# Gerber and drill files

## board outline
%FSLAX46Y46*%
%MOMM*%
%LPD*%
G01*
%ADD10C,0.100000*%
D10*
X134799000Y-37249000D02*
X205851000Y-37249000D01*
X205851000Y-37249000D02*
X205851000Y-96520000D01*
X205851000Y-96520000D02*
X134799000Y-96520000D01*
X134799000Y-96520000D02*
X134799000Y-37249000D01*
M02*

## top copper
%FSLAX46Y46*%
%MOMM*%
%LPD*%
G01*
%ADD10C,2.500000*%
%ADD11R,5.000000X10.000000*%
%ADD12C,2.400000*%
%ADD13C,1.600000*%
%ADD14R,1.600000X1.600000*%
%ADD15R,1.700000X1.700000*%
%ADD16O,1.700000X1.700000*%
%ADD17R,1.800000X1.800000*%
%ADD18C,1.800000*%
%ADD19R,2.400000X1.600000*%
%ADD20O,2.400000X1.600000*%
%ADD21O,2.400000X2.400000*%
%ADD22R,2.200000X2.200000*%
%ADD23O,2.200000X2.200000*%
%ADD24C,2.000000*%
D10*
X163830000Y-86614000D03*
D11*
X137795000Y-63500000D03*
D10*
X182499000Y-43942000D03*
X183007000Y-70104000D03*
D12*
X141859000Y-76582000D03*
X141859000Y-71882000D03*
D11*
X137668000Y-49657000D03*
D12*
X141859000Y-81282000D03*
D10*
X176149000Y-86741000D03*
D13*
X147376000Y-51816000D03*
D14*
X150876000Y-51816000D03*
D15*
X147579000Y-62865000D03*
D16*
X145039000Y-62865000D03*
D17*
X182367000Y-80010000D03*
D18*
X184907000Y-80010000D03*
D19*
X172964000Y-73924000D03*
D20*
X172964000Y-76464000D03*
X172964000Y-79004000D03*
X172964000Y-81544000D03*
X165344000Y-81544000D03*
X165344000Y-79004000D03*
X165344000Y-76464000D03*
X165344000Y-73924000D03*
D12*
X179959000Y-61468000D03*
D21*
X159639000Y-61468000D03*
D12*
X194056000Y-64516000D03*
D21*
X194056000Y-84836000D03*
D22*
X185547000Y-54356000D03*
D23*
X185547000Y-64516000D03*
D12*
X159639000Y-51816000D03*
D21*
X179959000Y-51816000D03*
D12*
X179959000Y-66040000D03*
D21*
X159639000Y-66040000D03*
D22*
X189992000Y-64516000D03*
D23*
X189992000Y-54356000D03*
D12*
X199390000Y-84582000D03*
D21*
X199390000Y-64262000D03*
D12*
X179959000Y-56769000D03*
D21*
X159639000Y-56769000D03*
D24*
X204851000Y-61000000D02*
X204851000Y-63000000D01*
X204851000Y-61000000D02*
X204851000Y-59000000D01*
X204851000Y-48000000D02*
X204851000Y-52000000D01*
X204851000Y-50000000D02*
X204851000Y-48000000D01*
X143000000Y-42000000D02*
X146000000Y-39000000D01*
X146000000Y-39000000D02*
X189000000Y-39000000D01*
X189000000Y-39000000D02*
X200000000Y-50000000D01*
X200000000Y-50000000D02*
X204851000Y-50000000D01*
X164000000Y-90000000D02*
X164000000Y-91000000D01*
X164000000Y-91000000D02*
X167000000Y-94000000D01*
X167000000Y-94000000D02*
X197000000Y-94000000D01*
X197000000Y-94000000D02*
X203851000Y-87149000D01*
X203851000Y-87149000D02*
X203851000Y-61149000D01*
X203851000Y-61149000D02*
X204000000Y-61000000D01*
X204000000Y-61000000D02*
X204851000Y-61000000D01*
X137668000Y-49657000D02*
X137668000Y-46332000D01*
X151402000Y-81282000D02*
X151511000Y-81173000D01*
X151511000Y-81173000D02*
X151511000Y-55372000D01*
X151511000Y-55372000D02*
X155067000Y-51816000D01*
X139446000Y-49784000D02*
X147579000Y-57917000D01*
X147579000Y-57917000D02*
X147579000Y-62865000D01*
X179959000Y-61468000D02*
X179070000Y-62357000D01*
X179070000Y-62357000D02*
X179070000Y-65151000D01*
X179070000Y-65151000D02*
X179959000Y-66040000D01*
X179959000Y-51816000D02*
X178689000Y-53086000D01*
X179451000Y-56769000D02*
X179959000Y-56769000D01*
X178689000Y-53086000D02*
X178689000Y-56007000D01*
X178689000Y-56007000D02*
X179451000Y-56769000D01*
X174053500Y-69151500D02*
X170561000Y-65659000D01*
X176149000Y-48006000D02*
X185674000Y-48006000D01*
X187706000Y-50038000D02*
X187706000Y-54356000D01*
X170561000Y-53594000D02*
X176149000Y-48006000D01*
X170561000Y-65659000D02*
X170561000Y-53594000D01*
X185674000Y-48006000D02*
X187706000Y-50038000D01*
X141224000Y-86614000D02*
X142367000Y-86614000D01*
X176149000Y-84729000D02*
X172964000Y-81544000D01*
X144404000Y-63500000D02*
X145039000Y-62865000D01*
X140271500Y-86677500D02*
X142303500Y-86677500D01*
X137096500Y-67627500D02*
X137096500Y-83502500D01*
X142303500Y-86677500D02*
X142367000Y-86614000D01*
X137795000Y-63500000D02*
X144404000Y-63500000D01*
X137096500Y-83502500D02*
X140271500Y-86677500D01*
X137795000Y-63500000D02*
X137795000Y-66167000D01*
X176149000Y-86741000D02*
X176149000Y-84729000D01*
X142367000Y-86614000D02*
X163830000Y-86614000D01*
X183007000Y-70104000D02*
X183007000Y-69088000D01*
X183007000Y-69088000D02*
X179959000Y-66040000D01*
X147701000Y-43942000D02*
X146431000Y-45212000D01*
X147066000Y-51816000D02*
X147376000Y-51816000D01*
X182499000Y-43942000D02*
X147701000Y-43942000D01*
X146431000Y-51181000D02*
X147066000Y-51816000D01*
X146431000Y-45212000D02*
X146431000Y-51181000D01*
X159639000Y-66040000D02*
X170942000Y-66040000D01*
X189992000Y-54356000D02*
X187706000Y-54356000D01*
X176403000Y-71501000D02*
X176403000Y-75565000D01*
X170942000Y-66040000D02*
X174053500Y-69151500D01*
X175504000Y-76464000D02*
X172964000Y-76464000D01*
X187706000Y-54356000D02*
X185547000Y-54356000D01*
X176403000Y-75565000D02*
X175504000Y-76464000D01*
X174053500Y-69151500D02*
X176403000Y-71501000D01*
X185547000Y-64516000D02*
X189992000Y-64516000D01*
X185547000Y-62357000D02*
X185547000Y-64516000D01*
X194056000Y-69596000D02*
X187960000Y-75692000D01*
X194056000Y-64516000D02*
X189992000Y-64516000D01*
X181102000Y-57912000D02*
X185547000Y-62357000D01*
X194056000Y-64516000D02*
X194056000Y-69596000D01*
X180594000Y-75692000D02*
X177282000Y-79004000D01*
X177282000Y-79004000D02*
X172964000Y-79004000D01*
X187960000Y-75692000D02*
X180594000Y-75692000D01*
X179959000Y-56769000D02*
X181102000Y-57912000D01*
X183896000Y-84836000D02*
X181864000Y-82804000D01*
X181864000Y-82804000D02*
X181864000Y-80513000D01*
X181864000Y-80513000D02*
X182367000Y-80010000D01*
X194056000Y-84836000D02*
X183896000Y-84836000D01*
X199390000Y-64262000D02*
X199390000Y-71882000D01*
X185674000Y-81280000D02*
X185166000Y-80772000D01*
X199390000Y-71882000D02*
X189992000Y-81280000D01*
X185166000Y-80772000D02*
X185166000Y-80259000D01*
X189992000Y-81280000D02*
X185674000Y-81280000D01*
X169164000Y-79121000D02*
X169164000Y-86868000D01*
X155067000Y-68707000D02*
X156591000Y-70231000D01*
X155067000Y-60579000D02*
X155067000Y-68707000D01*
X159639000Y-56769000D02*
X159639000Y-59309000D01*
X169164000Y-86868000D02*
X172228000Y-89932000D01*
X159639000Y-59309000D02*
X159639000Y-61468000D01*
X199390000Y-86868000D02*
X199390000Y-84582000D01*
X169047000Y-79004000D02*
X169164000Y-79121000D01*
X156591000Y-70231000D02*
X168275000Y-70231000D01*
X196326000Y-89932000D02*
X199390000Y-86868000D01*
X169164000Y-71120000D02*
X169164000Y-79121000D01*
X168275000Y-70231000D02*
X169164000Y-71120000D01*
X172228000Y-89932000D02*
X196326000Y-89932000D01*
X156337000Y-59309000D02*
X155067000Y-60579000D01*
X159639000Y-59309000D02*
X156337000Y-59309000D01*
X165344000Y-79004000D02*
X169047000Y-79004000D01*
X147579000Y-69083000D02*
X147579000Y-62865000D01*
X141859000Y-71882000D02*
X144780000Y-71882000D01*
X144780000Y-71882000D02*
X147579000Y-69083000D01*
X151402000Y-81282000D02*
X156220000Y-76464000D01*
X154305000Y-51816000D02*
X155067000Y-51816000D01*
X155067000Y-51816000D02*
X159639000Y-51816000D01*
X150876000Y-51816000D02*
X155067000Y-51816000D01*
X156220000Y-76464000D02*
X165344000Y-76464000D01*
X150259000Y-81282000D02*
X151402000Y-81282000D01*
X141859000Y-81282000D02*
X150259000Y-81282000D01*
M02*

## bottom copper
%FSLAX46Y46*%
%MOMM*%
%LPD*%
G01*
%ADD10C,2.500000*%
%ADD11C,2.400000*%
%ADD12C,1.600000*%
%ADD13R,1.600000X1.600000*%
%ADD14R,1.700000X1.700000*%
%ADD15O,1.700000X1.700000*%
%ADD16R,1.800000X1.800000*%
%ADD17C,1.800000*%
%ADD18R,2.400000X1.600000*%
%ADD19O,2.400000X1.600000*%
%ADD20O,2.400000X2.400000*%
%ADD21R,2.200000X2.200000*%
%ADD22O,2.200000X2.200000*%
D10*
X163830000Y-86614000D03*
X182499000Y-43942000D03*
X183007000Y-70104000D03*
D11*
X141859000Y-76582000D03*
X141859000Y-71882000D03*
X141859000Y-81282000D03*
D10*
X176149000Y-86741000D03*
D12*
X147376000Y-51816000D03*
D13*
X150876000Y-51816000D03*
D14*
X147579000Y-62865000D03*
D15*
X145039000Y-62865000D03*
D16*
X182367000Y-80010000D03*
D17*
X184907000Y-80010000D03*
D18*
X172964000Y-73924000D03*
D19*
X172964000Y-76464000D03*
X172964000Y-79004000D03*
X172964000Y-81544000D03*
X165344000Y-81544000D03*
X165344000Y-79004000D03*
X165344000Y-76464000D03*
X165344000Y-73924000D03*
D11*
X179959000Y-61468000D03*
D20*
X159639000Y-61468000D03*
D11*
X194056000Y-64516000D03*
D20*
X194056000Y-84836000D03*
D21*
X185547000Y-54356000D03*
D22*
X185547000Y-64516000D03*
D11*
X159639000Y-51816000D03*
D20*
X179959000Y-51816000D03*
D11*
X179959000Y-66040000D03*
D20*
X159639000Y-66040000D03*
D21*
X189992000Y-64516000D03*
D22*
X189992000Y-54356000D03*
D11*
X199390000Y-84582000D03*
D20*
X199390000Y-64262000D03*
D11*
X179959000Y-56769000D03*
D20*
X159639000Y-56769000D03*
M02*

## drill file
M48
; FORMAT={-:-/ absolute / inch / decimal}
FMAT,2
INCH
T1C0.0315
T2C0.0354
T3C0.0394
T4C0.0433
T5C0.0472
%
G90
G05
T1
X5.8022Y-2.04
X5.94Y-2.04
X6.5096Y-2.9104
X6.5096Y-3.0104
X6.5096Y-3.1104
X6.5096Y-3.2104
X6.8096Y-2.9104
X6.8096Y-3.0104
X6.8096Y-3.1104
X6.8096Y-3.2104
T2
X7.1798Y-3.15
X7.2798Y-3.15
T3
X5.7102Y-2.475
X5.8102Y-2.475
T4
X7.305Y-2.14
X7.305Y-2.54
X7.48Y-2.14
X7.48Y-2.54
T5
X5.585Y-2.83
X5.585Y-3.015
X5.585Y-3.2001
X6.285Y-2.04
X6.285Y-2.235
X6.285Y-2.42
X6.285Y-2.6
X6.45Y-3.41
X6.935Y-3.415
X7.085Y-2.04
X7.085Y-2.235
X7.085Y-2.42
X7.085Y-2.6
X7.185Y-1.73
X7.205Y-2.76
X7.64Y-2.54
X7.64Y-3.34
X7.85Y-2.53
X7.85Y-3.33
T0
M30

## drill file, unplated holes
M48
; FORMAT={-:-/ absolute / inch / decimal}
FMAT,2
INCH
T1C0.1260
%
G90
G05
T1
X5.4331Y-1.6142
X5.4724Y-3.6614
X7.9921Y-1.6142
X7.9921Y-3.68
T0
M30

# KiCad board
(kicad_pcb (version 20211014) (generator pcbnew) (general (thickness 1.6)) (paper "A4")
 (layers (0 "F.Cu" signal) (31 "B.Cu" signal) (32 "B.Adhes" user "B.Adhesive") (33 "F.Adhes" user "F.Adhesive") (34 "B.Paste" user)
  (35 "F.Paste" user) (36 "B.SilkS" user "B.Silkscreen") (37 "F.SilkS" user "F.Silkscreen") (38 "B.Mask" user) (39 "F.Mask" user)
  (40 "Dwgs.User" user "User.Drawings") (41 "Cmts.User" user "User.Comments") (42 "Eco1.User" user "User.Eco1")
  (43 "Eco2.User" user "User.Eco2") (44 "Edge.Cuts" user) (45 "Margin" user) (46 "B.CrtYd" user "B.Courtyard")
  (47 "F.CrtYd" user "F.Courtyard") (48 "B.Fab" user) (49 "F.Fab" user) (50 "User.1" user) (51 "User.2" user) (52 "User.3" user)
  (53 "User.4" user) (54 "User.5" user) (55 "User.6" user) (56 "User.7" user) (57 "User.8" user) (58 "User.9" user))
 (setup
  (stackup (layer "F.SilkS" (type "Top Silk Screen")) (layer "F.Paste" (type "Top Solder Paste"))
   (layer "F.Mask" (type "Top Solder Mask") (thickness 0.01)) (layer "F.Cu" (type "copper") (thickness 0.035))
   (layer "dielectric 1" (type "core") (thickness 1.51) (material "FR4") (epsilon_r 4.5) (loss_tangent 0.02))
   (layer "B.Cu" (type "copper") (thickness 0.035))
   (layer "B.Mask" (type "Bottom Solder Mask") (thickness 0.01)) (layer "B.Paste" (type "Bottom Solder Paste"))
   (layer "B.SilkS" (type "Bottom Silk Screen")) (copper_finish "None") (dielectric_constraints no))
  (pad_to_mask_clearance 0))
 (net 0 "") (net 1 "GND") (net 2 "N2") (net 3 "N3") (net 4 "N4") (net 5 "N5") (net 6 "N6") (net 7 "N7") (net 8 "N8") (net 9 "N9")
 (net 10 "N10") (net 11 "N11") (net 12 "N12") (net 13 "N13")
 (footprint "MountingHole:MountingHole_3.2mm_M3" (layer "F.Cu") (at 138 41)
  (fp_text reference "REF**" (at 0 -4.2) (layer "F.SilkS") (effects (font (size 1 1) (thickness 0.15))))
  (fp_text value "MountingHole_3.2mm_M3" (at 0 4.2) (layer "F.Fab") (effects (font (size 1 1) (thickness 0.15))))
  (pad "" np_thru_hole circle (at 0 0) (size 3.2 3.2) (drill 3.2) (layers F&B.Cu *.Mask)))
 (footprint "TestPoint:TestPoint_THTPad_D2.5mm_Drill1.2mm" (layer "F.Cu") (at 163.83 86.614)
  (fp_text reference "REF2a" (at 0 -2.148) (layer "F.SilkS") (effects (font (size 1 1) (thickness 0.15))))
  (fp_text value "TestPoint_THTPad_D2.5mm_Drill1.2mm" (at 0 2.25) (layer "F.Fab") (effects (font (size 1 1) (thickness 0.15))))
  (pad "1" thru_hole circle (at 0 0) (size 2.5 2.5) (drill 1.2) (layers *.Cu *.Mask) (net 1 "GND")))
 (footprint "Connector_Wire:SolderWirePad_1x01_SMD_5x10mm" (layer "F.Cu") (at 137.795 63.5)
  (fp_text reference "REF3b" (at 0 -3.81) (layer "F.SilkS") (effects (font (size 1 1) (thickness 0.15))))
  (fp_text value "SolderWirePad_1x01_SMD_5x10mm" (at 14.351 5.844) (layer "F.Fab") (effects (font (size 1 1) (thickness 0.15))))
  (pad "1" smd rect (at 0 0) (size 5 10) (layers "F.Cu" "F.Paste" "F.Mask") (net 1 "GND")))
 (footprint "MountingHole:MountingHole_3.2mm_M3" (layer "F.Cu") (at 139 93)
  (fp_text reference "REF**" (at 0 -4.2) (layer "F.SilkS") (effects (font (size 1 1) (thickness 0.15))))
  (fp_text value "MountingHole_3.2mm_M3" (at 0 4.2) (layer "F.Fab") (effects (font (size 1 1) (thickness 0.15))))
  (pad "" np_thru_hole circle (at 0 0) (size 3.2 3.2) (drill 3.2) (layers F&B.Cu *.Mask)))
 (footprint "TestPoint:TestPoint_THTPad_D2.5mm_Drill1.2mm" (layer "F.Cu") (at 182.499 43.942)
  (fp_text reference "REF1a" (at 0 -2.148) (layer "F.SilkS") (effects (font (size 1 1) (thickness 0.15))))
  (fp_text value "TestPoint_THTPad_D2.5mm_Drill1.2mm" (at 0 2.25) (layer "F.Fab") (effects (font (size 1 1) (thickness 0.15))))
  (pad "1" thru_hole circle (at 0 0) (size 2.5 2.5) (drill 1.2) (layers *.Cu *.Mask) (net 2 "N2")))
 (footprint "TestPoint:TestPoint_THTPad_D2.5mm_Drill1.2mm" (layer "F.Cu") (at 183.007 70.104)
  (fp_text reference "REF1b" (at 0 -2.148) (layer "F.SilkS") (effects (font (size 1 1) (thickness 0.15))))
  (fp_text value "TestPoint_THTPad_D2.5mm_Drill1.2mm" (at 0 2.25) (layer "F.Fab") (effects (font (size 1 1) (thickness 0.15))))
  (pad "1" thru_hole circle (at 0 0) (size 2.5 2.5) (drill 1.2) (layers *.Cu *.Mask) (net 2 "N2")))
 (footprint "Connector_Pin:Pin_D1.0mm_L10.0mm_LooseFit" (layer "F.Cu") (at 141.859 76.582 90)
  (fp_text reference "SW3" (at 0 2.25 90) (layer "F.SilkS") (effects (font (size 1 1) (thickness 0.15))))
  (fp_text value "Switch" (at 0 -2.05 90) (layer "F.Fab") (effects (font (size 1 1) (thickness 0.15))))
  (pad "1" thru_hole circle (at 0 0 90) (size 2.4 2.4) (drill 1.2) (layers *.Cu *.Mask) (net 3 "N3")))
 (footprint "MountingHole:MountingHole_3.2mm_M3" (layer "F.Cu") (at 203 93.472)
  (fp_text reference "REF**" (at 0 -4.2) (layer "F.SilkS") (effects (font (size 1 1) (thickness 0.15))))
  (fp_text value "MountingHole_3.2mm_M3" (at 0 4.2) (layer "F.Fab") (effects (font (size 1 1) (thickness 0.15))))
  (pad "" np_thru_hole circle (at 0 0) (size 3.2 3.2) (drill 3.2) (layers *.Cu *.Mask)))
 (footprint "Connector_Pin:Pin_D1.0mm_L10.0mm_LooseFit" (layer "F.Cu") (at 141.859 71.882 90)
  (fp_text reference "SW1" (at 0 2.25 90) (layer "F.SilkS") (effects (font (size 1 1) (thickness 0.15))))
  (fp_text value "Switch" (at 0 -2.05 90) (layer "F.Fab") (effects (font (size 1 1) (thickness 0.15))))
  (pad "1" thru_hole circle (at 0 0 90) (size 2.4 2.4) (drill 1.2) (layers *.Cu *.Mask) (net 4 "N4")))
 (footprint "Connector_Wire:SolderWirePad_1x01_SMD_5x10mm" (layer "F.Cu") (at 137.668 49.657)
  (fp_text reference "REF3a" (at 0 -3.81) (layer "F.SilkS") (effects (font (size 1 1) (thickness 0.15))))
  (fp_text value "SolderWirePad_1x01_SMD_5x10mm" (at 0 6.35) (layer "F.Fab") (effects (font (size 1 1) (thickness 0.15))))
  (pad "1" smd rect (at 0 0) (size 5 10) (layers "F.Cu" "F.Paste" "F.Mask") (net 4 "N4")))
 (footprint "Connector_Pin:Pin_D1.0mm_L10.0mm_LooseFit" (layer "F.Cu") (at 141.859 81.282 90)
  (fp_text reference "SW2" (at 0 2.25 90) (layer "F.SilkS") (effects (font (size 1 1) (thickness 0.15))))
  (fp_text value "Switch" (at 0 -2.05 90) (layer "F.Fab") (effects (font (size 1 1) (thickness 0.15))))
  (pad "1" thru_hole circle (at 0 0 90) (size 2.4 2.4) (drill 1.2) (layers *.Cu *.Mask) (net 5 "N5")))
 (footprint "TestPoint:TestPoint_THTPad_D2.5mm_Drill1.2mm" (layer "F.Cu") (at 176.149 86.741)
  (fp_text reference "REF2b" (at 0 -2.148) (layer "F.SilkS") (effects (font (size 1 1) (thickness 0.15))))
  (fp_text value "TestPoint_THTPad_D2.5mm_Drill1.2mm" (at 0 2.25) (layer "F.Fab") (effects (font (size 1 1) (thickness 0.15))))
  (pad "1" thru_hole circle (at 0 0) (size 2.5 2.5) (drill 1.2) (layers *.Cu *.Mask) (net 1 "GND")))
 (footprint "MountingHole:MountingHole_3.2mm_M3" (layer "F.Cu") (at 203 41)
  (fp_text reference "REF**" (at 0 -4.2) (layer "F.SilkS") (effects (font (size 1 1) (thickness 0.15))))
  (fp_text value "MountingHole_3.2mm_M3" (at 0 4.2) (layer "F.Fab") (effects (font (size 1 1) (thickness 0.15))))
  (pad "" np_thru_hole circle (at 0 0) (size 3.2 3.2) (drill 3.2) (layers F&B.Cu *.Mask)))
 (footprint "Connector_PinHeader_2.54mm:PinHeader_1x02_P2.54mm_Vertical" (layer "B.Cu") (at 147.579 62.865 90)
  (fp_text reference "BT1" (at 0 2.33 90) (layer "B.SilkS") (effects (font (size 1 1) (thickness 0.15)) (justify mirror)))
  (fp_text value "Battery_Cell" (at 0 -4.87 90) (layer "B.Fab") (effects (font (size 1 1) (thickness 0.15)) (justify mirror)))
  (pad "1" thru_hole rect (at 0 0 90) (size 1.7 1.7) (drill 1) (layers *.Cu *.Mask) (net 4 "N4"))
  (pad "2" thru_hole oval (at 0 -2.54 90) (size 1.7 1.7) (drill 1) (layers *.Cu *.Mask) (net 1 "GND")))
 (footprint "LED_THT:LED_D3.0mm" (layer "B.Cu") (at 182.367 80.01)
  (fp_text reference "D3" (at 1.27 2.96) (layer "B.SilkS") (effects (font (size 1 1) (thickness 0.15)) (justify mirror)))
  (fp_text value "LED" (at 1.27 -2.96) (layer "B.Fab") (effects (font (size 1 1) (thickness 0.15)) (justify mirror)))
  (pad "1" thru_hole rect (at 0 0) (size 1.8 1.8) (drill 0.9) (layers *.Cu *.Mask) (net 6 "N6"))
  (pad "2" thru_hole circle (at 2.54 0) (size 1.8 1.8) (drill 0.9) (layers *.Cu *.Mask) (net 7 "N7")))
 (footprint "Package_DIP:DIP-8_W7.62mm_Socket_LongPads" (layer "B.Cu") (at 172.964 73.924 180)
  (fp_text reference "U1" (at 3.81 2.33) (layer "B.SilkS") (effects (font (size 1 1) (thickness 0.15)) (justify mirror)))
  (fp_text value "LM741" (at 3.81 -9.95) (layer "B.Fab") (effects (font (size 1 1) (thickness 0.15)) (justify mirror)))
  (pad "1" thru_hole rect (at 0 0 180) (size 2.4 1.6) (drill 0.8) (layers *.Cu *.Mask) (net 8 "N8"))
  (pad "2" thru_hole oval (at 0 -2.54 180) (size 2.4 1.6) (drill 0.8) (layers *.Cu *.Mask) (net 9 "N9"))
  (pad "3" thru_hole oval (at 0 -5.08 180) (size 2.4 1.6) (drill 0.8) (layers *.Cu *.Mask) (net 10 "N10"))
  (pad "4" thru_hole oval (at 0 -7.62 180) (size 2.4 1.6) (drill 0.8) (layers *.Cu *.Mask) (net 1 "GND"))
  (pad "5" thru_hole oval (at 7.62 -7.62 180) (size 2.4 1.6) (drill 0.8) (layers *.Cu *.Mask) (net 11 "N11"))
  (pad "6" thru_hole oval (at 7.62 -5.08 180) (size 2.4 1.6) (drill 0.8) (layers *.Cu *.Mask) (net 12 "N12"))
  (pad "7" thru_hole oval (at 7.62 -2.54 180) (size 2.4 1.6) (drill 0.8) (layers *.Cu *.Mask) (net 5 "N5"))
  (pad "8" thru_hole oval (at 7.62 0 180) (size 2.4 1.6) (drill 0.8) (layers *.Cu *.Mask) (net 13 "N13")))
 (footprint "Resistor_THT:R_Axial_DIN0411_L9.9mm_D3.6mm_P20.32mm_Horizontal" (layer "B.Cu") (at 179.959 61.468 180)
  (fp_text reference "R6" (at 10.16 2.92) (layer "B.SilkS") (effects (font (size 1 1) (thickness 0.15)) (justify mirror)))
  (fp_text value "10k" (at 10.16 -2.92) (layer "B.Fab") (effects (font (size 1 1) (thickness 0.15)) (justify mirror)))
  (pad "1" thru_hole circle (at 0 0 180) (size 2.4 2.4) (drill 1.2) (layers *.Cu *.Mask) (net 2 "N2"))
  (pad "2" thru_hole oval (at 20.32 0 180) (size 2.4 2.4) (drill 1.2) (layers *.Cu *.Mask) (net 12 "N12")))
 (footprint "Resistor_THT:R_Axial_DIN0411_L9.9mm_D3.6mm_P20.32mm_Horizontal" (layer "B.Cu") (at 194.056 64.516 -90)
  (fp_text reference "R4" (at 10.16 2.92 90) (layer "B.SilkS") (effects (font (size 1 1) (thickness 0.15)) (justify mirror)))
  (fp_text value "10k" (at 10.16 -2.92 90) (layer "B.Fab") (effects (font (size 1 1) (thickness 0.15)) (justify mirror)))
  (pad "1" thru_hole circle (at 0 0 270) (size 2.4 2.4) (drill 1.2) (layers *.Cu *.Mask) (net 10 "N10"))
  (pad "2" thru_hole oval (at 20.32 0 270) (size 2.4 2.4) (drill 1.2) (layers *.Cu *.Mask) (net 6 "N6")))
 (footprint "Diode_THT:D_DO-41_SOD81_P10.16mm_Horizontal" (layer "B.Cu") (at 185.547 54.356 -90)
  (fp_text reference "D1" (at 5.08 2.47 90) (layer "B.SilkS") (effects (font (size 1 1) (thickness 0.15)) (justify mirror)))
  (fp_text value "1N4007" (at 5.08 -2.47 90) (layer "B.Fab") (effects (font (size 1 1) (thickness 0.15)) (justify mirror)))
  (pad "1" thru_hole rect (at 0 0 270) (size 2.2 2.2) (drill 1.1) (layers *.Cu *.Mask) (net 9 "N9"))
  (pad "2" thru_hole oval (at 10.16 0 270) (size 2.2 2.2) (drill 1.1) (layers *.Cu *.Mask) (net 10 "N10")))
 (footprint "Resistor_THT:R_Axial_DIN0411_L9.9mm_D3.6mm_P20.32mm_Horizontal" (layer "B.Cu") (at 159.639 51.816)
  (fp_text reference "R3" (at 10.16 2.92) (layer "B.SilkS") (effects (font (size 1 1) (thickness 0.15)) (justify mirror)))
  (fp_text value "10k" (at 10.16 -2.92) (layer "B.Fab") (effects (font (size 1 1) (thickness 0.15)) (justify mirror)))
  (pad "1" thru_hole circle (at 0 0) (size 2.4 2.4) (drill 1.2) (layers *.Cu *.Mask) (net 5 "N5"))
  (pad "2" thru_hole oval (at 20.32 0) (size 2.4 2.4) (drill 1.2) (layers *.Cu *.Mask) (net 10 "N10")))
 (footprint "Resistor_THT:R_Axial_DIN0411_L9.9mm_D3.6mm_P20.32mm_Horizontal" (layer "B.Cu") (at 179.959 66.04 180)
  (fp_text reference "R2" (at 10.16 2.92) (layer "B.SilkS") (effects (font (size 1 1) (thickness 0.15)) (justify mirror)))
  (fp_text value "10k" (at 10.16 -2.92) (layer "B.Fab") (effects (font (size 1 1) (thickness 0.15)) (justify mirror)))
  (pad "1" thru_hole circle (at 0 0 180) (size 2.4 2.4) (drill 1.2) (layers *.Cu *.Mask) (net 2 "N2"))
  (pad "2" thru_hole oval (at 20.32 0 180) (size 2.4 2.4) (drill 1.2) (layers *.Cu *.Mask) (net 9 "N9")))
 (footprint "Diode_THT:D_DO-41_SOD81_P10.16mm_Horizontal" (layer "B.Cu") (at 189.992 64.516 90)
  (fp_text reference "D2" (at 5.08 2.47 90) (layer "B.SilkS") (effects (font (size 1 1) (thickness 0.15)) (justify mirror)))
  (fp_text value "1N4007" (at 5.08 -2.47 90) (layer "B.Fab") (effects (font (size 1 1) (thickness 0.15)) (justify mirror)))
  (pad "1" thru_hole rect (at 0 0 90) (size 2.2 2.2) (drill 1.1) (layers *.Cu *.Mask) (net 10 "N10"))
  (pad "2" thru_hole oval (at 10.16 0 90) (size 2.2 2.2) (drill 1.1) (layers *.Cu *.Mask) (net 9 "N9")))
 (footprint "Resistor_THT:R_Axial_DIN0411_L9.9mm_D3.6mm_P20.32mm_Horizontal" (layer "B.Cu") (at 199.39 84.582 90)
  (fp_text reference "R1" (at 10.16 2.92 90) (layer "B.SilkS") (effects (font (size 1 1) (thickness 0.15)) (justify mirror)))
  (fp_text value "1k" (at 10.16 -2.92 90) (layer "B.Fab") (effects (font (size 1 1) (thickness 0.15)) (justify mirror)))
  (pad "1" thru_hole circle (at 0 0 90) (size 2.4 2.4) (drill 1.2) (layers *.Cu *.Mask) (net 12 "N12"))
  (pad "2" thru_hole oval (at 20.32 0 90) (size 2.4 2.4) (drill 1.2) (layers *.Cu *.Mask) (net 7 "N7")))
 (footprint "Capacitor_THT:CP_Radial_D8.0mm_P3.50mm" (layer "B.Cu") (at 150.876 51.816 180)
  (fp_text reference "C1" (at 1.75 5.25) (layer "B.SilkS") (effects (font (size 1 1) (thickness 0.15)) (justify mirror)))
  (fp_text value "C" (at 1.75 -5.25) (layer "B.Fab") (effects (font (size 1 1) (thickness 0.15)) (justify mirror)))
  (pad "1" thru_hole rect (at 0 0 180) (size 1.6 1.6) (drill 0.8) (layers *.Cu *.Mask) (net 5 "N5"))
  (pad "2" thru_hole circle (at 3.5 0 180) (size 1.6 1.6) (drill 0.8) (layers *.Cu *.Mask) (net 2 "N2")))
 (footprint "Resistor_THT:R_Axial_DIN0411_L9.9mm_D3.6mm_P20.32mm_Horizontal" (layer "B.Cu") (at 179.959 56.769 180)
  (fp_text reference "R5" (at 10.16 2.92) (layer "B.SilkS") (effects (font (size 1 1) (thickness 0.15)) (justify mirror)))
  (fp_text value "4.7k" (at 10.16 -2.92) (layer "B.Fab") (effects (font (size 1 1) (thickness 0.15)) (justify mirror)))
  (pad "1" thru_hole circle (at 0 0 180) (size 2.4 2.4) (drill 1.2) (layers *.Cu *.Mask) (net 10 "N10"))
  (pad "2" thru_hole oval (at 20.32 0 180) (size 2.4 2.4) (drill 1.2) (layers *.Cu *.Mask) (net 12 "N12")))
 (gr_rect (start 134.799 37.249) (end 205.851 96.52) (layer "Edge.Cuts") (width 0.1) (fill none))
 (segment (start 204.851 61) (end 204.851 63) (width 2) (layer "F.Cu") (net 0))
 (segment (start 197 94) (end 203.851 87.149) (width 2) (layer "F.Cu") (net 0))
 (segment (start 203.851 61.149) (end 204 61) (width 2) (layer "F.Cu") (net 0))
 (segment (start 164 91) (end 167 94) (width 2) (layer "F.Cu") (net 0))
 (segment (start 203.851 87.149) (end 203.851 61.149) (width 2) (layer "F.Cu") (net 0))
 (segment (start 164 90) (end 164 91) (width 2) (layer "F.Cu") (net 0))
 (segment (start 204.851 61) (end 204.851 59) (width 2) (layer "F.Cu") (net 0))
 (segment (start 167 94) (end 197 94) (width 2) (layer "F.Cu") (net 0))
 (segment (start 204 61) (end 204.851 61) (width 2) (layer "F.Cu") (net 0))
 (segment (start 141.224 86.614) (end 142.367 86.614) (width 2) (layer "F.Cu") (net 1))
 (segment (start 176.149 84.729) (end 172.964 81.544) (width 2) (layer "F.Cu") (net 1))
 (segment (start 144.404 63.5) (end 145.039 62.865) (width 2) (layer "F.Cu") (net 1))
 (segment (start 140.2715 86.6775) (end 142.3035 86.6775) (width 2) (layer "F.Cu") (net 1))
 (segment (start 137.0965 67.6275) (end 137.0965 83.5025) (width 2) (layer "F.Cu") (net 1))
 (segment (start 142.3035 86.6775) (end 142.367 86.614) (width 2) (layer "F.Cu") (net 1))
 (segment (start 137.795 63.5) (end 144.404 63.5) (width 2) (layer "F.Cu") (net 1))
 (segment (start 137.0965 83.5025) (end 140.2715 86.6775) (width 2) (layer "F.Cu") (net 1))
 (segment (start 137.795 63.5) (end 137.795 66.167) (width 2) (layer "F.Cu") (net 1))
 (segment (start 176.149 86.741) (end 176.149 84.729) (width 2) (layer "F.Cu") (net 1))
 (segment (start 142.367 86.614) (end 163.83 86.614) (width 2) (layer "F.Cu") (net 1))
 (segment (start 183.007 70.104) (end 183.007 69.088) (width 2) (layer "F.Cu") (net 2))
 (segment (start 183.007 69.088) (end 179.959 66.04) (width 2) (layer "F.Cu") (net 2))
 (segment (start 147.701 43.942) (end 146.431 45.212) (width 2) (layer "F.Cu") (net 2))
 (segment (start 179.07 62.357) (end 179.07 65.151) (width 2) (layer "F.Cu") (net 2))
 (segment (start 147.066 51.816) (end 147.376 51.816) (width 2) (layer "F.Cu") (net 2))
 (segment (start 182.499 43.942) (end 147.701 43.942) (width 2) (layer "F.Cu") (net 2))
 (segment (start 179.959 61.468) (end 179.07 62.357) (width 2) (layer "F.Cu") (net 2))
 (segment (start 146.431 51.181) (end 147.066 51.816) (width 2) (layer "F.Cu") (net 2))
 (segment (start 179.07 65.151) (end 179.959 66.04) (width 2) (layer "F.Cu") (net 2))
 (segment (start 146.431 45.212) (end 146.431 51.181) (width 2) (layer "F.Cu") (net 2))
 (segment (start 159.639 66.04) (end 170.942 66.04) (width 2) (layer "F.Cu") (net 9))
 (segment (start 174.0535 69.1515) (end 170.561 65.659) (width 2) (layer "F.Cu") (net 9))
 (segment (start 170.561 53.594) (end 176.149 48.006) (width 2) (layer "F.Cu") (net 9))
 (segment (start 189.992 54.356) (end 187.706 54.356) (width 2) (layer "F.Cu") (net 9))
 (segment (start 185.674 48.006) (end 187.706 50.038) (width 2) (layer "F.Cu") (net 9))
 (segment (start 176.403 71.501) (end 176.403 75.565) (width 2) (layer "F.Cu") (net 9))
 (segment (start 170.561 65.659) (end 170.561 53.594) (width 2) (layer "F.Cu") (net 9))
 (segment (start 170.942 66.04) (end 174.0535 69.1515) (width 2) (layer "F.Cu") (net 9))
 (segment (start 175.504 76.464) (end 172.964 76.464) (width 2) (layer "F.Cu") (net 9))
 (segment (start 187.706 50.038) (end 187.706 54.356) (width 2) (layer "F.Cu") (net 9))
 (segment (start 187.706 54.356) (end 185.547 54.356) (width 2) (layer "F.Cu") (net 9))
 (segment (start 176.403 75.565) (end 175.504 76.464) (width 2) (layer "F.Cu") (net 9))
 (segment (start 176.149 48.006) (end 185.674 48.006) (width 2) (layer "F.Cu") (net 9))
 (segment (start 174.0535 69.1515) (end 176.403 71.501) (width 2) (layer "F.Cu") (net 9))
 (segment (start 179.959 51.816) (end 178.689 53.086) (width 2) (layer "F.Cu") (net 10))
 (segment (start 185.547 64.516) (end 189.992 64.516) (width 2) (layer "F.Cu") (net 10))
 (segment (start 185.547 62.357) (end 185.547 64.516) (width 2) (layer "F.Cu") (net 10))
 (segment (start 194.056 69.596) (end 187.96 75.692) (width 2) (layer "F.Cu") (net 10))
 (segment (start 194.056 64.516) (end 189.992 64.516) (width 2) (layer "F.Cu") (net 10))
 (segment (start 181.102 57.912) (end 185.547 62.357) (width 2) (layer "F.Cu") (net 10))
 (segment (start 178.689 53.086) (end 178.689 56.007) (width 2) (layer "F.Cu") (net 10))
 (segment (start 194.056 64.516) (end 194.056 69.596) (width 2) (layer "F.Cu") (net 10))
 (segment (start 180.594 75.692) (end 177.282 79.004) (width 2) (layer "F.Cu") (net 10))
 (segment (start 179.451 56.769) (end 179.959 56.769) (width 2) (layer "F.Cu") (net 10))
 (segment (start 178.689 56.007) (end 179.451 56.769) (width 2) (layer "F.Cu") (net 10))
 (segment (start 177.282 79.004) (end 172.964 79.004) (width 2) (layer "F.Cu") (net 10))
 (segment (start 187.96 75.692) (end 180.594 75.692) (width 2) (layer "F.Cu") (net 10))
 (segment (start 179.959 56.769) (end 181.102 57.912) (width 2) (layer "F.Cu") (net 10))
 (segment (start 183.896 84.836) (end 181.864 82.804) (width 2) (layer "F.Cu") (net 6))
 (segment (start 181.864 82.804) (end 181.864 80.513) (width 2) (layer "F.Cu") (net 6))
 (segment (start 181.864 80.513) (end 182.367 80.01) (width 2) (layer "F.Cu") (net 6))
 (segment (start 194.056 84.836) (end 183.896 84.836) (width 2) (layer "F.Cu") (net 6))
 (segment (start 199.39 64.262) (end 199.39 71.882) (width 2) (layer "F.Cu") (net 7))
 (segment (start 185.674 81.28) (end 185.166 80.772) (width 2) (layer "F.Cu") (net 7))
 (segment (start 199.39 71.882) (end 189.992 81.28) (width 2) (layer "F.Cu") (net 7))
 (segment (start 185.166 80.772) (end 185.166 80.259) (width 2) (layer "F.Cu") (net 7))
 (segment (start 189.992 81.28) (end 185.674 81.28) (width 2) (layer "F.Cu") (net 7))
 (segment (start 169.164 79.121) (end 169.164 86.868) (width 2) (layer "F.Cu") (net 12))
 (segment (start 155.067 68.707) (end 156.591 70.231) (width 2) (layer "F.Cu") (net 12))
 (segment (start 155.067 60.579) (end 155.067 68.707) (width 2) (layer "F.Cu") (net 12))
 (segment (start 159.639 56.769) (end 159.639 59.309) (width 2) (layer "F.Cu") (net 12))
 (segment (start 169.164 86.868) (end 172.228 89.932) (width 2) (layer "F.Cu") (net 12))
 (segment (start 159.639 59.309) (end 159.639 61.468) (width 2) (layer "F.Cu") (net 12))
 (segment (start 199.39 86.868) (end 199.39 84.582) (width 2) (layer "F.Cu") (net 12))
 (segment (start 169.047 79.004) (end 169.164 79.121) (width 2) (layer "F.Cu") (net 12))
 (segment (start 156.591 70.231) (end 168.275 70.231) (width 2) (layer "F.Cu") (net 12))
 (segment (start 196.326 89.932) (end 199.39 86.868) (width 2) (layer "F.Cu") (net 12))
 (segment (start 169.164 71.12) (end 169.164 79.121) (width 2) (layer "F.Cu") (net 12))
 (segment (start 168.275 70.231) (end 169.164 71.12) (width 2) (layer "F.Cu") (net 12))
 (segment (start 172.228 89.932) (end 196.326 89.932) (width 2) (layer "F.Cu") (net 12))
 (segment (start 156.337 59.309) (end 155.067 60.579) (width 2) (layer "F.Cu") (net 12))
 (segment (start 159.639 59.309) (end 156.337 59.309) (width 2) (layer "F.Cu") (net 12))
 (segment (start 165.344 79.004) (end 169.047 79.004) (width 2) (layer "F.Cu") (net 12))
 (segment (start 189 39) (end 200 50) (width 2) (layer "F.Cu") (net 4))
 (segment (start 147.579 57.917) (end 147.579 62.865) (width 2) (layer "F.Cu") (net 4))
 (segment (start 200 50) (end 204.851 50) (width 2) (layer "F.Cu") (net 4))
 (segment (start 147.579 69.083) (end 147.579 62.865) (width 2) (layer "F.Cu") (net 4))
 (segment (start 141.859 71.882) (end 144.78 71.882) (width 2) (layer "F.Cu") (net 4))
 (segment (start 204.851 50) (end 204.851 48) (width 2) (layer "F.Cu") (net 4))
 (segment (start 204.851 48) (end 204.851 52) (width 2) (layer "F.Cu") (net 4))
 (segment (start 146 39) (end 189 39) (width 2) (layer "F.Cu") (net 4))
 (segment (start 144.78 71.882) (end 147.579 69.083) (width 2) (layer "F.Cu") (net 4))
 (segment (start 139.446 49.784) (end 147.579 57.917) (width 2) (layer "F.Cu") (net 4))
 (segment (start 137.668 49.657) (end 137.668 46.332) (width 2) (layer "F.Cu") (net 4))
 (segment (start 143 42) (end 146 39) (width 2) (layer "F.Cu") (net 4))
 (segment (start 151.402 81.282) (end 156.22 76.464) (width 2) (layer "F.Cu") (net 5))
 (segment (start 151.402 81.282) (end 151.511 81.173) (width 2) (layer "F.Cu") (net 5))
 (segment (start 154.305 51.816) (end 155.067 51.816) (width 2) (layer "F.Cu") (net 5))
 (segment (start 151.511 81.173) (end 151.511 55.372) (width 2) (layer "F.Cu") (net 5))
 (segment (start 151.511 55.372) (end 155.067 51.816) (width 2) (layer "F.Cu") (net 5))
 (segment (start 155.067 51.816) (end 159.639 51.816) (width 2) (layer "F.Cu") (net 5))
 (segment (start 150.876 51.816) (end 155.067 51.816) (width 2) (layer "F.Cu") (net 5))
 (segment (start 156.22 76.464) (end 165.344 76.464) (width 2) (layer "F.Cu") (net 5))
 (segment (start 150.259 81.282) (end 151.402 81.282) (width 2) (layer "F.Cu") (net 5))
 (segment (start 141.859 81.282) (end 150.259 81.282) (width 2) (layer "F.Cu") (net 5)))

